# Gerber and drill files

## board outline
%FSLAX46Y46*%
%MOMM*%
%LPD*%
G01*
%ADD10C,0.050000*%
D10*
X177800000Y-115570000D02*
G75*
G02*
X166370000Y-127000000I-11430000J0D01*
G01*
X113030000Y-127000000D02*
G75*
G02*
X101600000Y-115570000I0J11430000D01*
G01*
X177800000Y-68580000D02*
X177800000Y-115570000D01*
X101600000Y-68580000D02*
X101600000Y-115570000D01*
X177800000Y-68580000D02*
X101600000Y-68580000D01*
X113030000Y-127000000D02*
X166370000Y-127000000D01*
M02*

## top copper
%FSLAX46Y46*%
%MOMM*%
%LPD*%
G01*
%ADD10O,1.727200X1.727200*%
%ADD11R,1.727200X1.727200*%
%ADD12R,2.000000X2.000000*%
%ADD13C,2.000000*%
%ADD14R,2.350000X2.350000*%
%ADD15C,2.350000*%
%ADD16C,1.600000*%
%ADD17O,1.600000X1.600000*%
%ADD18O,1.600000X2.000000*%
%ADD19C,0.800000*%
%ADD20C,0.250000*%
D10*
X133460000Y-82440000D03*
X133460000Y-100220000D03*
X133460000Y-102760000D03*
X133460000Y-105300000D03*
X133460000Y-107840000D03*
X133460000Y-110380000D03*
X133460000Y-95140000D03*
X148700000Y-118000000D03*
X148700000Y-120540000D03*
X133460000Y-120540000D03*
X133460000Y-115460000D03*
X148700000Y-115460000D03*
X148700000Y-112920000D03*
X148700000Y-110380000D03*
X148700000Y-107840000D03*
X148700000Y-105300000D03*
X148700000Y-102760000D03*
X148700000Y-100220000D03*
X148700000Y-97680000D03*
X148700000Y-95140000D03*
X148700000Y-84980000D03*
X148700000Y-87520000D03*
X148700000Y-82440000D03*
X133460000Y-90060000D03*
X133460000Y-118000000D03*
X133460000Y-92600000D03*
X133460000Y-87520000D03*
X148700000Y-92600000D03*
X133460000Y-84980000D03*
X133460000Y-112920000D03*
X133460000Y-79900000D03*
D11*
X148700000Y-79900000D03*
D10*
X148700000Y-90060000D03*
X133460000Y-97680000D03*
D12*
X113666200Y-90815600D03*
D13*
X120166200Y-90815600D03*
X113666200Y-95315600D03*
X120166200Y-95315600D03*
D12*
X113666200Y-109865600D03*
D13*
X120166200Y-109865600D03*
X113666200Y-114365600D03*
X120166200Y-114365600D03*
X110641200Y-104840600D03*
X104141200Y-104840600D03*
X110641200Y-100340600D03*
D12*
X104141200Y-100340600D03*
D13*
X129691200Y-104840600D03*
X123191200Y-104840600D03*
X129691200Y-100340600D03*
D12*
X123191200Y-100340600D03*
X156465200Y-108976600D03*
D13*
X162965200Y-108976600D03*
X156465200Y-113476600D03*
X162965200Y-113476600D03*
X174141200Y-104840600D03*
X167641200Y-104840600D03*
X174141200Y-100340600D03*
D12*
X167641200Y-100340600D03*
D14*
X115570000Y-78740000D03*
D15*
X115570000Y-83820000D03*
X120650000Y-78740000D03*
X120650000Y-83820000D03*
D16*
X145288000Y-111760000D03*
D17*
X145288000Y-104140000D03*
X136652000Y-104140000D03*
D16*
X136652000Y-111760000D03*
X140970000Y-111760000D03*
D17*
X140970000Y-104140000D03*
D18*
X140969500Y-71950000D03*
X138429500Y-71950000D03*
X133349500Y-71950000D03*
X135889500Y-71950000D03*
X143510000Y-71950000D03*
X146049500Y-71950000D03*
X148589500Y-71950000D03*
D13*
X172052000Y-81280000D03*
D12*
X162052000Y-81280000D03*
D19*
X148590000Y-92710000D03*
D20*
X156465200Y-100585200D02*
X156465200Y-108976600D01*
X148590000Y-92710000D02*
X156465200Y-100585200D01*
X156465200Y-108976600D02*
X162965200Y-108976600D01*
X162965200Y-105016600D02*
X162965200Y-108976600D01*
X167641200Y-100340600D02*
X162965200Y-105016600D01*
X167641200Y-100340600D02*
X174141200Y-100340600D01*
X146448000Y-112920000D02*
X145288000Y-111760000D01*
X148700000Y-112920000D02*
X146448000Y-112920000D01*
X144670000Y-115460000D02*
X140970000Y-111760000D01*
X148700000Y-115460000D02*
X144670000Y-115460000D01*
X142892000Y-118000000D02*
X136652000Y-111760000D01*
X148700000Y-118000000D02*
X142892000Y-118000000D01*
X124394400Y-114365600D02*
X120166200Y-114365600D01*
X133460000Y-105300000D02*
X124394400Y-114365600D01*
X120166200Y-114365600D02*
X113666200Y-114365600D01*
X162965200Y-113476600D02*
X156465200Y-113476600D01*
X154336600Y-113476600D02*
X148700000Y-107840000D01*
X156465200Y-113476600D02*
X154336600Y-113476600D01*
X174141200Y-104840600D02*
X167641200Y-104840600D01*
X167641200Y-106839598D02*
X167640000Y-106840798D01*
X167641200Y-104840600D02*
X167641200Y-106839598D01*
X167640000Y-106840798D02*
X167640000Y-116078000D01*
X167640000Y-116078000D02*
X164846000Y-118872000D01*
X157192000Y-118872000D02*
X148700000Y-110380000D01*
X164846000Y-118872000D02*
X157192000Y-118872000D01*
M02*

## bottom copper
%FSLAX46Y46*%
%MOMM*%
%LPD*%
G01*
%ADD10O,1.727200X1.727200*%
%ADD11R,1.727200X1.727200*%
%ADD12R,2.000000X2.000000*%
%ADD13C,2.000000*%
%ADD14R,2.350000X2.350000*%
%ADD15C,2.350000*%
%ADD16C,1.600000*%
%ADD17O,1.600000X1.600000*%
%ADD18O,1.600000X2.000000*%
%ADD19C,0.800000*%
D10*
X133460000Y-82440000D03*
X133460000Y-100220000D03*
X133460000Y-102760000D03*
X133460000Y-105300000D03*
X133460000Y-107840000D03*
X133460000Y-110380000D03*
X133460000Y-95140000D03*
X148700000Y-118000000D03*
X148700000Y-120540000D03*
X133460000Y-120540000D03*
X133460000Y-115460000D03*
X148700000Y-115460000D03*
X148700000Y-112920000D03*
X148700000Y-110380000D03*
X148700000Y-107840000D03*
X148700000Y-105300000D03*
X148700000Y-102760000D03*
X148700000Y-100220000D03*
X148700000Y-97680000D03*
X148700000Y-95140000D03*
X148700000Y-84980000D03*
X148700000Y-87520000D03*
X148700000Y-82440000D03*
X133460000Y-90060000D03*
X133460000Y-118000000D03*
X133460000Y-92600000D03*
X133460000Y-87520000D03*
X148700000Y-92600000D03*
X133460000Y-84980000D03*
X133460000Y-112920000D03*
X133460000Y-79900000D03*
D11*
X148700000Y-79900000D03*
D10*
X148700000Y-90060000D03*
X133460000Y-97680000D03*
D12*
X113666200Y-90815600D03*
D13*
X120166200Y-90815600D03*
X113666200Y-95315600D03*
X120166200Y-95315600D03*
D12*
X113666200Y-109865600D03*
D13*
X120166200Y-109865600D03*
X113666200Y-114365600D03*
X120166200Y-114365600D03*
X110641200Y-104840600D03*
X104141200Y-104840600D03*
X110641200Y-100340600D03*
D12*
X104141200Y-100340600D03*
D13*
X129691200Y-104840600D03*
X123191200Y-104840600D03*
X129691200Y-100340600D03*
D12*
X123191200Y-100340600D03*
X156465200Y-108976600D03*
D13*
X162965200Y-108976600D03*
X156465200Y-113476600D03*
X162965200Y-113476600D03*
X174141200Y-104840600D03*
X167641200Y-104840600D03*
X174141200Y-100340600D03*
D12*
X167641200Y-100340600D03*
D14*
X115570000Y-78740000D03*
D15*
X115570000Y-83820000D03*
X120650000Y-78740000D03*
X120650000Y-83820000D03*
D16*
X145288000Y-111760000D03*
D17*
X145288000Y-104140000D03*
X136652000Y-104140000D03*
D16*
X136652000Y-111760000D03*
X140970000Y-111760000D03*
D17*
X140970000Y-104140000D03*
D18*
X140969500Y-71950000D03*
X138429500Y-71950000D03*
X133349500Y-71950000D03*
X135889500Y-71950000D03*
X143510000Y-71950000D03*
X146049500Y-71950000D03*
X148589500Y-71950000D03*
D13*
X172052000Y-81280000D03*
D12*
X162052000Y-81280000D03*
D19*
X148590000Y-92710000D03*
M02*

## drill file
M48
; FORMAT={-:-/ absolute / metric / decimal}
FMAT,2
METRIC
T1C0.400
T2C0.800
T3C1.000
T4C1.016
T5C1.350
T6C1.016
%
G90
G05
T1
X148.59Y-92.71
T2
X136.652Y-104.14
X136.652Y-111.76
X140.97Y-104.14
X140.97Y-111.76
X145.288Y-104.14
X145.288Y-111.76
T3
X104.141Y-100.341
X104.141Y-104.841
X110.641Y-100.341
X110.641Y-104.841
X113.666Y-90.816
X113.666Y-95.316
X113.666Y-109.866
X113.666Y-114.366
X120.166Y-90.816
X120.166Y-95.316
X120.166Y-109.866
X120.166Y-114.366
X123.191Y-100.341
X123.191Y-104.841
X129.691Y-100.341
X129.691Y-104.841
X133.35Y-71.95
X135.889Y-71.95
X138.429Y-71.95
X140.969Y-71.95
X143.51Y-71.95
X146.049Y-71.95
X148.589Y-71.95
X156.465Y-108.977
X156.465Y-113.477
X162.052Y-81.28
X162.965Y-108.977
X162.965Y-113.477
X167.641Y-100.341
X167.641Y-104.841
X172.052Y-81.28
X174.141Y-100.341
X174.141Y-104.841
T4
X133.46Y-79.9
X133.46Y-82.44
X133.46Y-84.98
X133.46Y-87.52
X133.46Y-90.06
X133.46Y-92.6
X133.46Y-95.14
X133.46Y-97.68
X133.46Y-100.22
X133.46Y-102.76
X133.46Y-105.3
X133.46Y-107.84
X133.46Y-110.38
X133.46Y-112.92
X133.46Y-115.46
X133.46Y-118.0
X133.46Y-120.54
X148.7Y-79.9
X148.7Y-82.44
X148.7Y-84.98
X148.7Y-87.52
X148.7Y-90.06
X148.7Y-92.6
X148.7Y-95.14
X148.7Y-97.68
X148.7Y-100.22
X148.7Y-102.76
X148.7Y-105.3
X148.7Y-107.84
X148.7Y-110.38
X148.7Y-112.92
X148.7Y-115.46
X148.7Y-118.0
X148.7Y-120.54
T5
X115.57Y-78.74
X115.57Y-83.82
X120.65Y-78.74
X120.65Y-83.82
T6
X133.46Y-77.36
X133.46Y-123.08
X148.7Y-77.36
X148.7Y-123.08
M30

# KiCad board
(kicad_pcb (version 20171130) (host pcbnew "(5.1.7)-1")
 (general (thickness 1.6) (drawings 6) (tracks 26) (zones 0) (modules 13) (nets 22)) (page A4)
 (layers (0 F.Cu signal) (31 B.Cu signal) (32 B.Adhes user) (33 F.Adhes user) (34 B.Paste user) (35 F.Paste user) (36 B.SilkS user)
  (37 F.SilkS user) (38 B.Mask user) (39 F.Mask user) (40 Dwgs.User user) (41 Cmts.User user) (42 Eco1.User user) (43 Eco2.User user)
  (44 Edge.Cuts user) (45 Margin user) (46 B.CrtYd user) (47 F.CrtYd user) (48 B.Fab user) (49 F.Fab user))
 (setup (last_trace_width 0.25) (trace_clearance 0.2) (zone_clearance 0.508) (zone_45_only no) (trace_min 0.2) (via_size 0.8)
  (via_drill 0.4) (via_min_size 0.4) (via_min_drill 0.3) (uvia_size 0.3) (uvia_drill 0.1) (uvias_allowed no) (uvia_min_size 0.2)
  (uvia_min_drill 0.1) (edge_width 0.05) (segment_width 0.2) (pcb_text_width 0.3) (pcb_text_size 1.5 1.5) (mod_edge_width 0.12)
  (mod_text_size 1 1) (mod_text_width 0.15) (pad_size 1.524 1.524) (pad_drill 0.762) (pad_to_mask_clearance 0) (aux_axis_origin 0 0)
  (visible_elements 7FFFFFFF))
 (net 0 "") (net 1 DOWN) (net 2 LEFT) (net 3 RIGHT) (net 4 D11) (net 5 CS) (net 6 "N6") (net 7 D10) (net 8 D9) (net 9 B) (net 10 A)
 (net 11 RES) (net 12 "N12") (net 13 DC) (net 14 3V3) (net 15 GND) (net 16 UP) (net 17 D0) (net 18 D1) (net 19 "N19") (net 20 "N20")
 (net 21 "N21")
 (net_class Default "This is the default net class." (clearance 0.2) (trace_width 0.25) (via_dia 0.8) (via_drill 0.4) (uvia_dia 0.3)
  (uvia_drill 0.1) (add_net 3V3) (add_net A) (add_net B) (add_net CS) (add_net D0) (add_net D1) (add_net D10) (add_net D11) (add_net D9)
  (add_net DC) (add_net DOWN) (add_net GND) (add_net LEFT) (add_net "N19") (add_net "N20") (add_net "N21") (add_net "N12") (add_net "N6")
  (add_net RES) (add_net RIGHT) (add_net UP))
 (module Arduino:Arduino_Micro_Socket (layer B.Cu) (at 132.08 124.46 90)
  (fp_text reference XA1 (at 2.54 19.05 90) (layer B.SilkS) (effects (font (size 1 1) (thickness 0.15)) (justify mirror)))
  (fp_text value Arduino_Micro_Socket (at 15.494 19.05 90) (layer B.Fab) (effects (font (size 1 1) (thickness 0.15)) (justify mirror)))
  (pad MISO thru_hole oval (at 42.02 1.38 90) (size 1.7272 1.7272) (drill 1.016) (layers *.Cu *.Mask))
  (pad A5 thru_hole oval (at 24.24 1.38 90) (size 1.7272 1.7272) (drill 1.016) (layers *.Cu *.Mask))
  (pad A4 thru_hole oval (at 21.7 1.38 90) (size 1.7272 1.7272) (drill 1.016) (layers *.Cu *.Mask))
  (pad A3 thru_hole oval (at 19.16 1.38 90) (size 1.7272 1.7272) (drill 1.016) (layers *.Cu *.Mask) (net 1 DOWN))
  (pad A2 thru_hole oval (at 16.62 1.38 90) (size 1.7272 1.7272) (drill 1.016) (layers *.Cu *.Mask) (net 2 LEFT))
  (pad A1 thru_hole oval (at 14.08 1.38 90) (size 1.7272 1.7272) (drill 1.016) (layers *.Cu *.Mask) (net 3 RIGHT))
  (pad "" thru_hole oval (at 29.32 1.38 90) (size 1.7272 1.7272) (drill 1.016) (layers *.Cu *.Mask))
  (pad D11 thru_hole oval (at 6.46 16.62 90) (size 1.7272 1.7272) (drill 1.016) (layers *.Cu *.Mask) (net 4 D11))
  (pad D12 thru_hole oval (at 3.92 16.62 90) (size 1.7272 1.7272) (drill 1.016) (layers *.Cu *.Mask) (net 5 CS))
  (pad D13 thru_hole oval (at 3.92 1.38 90) (size 1.7272 1.7272) (drill 1.016) (layers *.Cu *.Mask) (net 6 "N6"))
  (pad AREF thru_hole oval (at 9 1.38 90) (size 1.7272 1.7272) (drill 1.016) (layers *.Cu *.Mask))
  (pad "" np_thru_hole circle (at 1.38 1.38 90) (size 1.016 1.016) (drill 1.016) (layers *.Cu *.Mask))
  (pad D10 thru_hole oval (at 9 16.62 90) (size 1.7272 1.7272) (drill 1.016) (layers *.Cu *.Mask) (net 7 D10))
  (pad D9 thru_hole oval (at 11.54 16.62 90) (size 1.7272 1.7272) (drill 1.016) (layers *.Cu *.Mask) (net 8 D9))
  (pad D8 thru_hole oval (at 14.08 16.62 90) (size 1.7272 1.7272) (drill 1.016) (layers *.Cu *.Mask) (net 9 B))
  (pad D7 thru_hole oval (at 16.62 16.62 90) (size 1.7272 1.7272) (drill 1.016) (layers *.Cu *.Mask) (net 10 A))
  (pad D6 thru_hole oval (at 19.16 16.62 90) (size 1.7272 1.7272) (drill 1.016) (layers *.Cu *.Mask) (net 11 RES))
  (pad D5 thru_hole oval (at 21.7 16.62 90) (size 1.7272 1.7272) (drill 1.016) (layers *.Cu *.Mask) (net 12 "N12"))
  (pad D4 thru_hole oval (at 24.24 16.62 90) (size 1.7272 1.7272) (drill 1.016) (layers *.Cu *.Mask) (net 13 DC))
  (pad D3 thru_hole oval (at 26.78 16.62 90) (size 1.7272 1.7272) (drill 1.016) (layers *.Cu *.Mask))
  (pad D2 thru_hole oval (at 29.32 16.62 90) (size 1.7272 1.7272) (drill 1.016) (layers *.Cu *.Mask))
  (pad D1 thru_hole oval (at 39.48 16.62 90) (size 1.7272 1.7272) (drill 1.016) (layers *.Cu *.Mask))
  (pad D0 thru_hole oval (at 36.94 16.62 90) (size 1.7272 1.7272) (drill 1.016) (layers *.Cu *.Mask))
  (pad SS thru_hole oval (at 42.02 16.62 90) (size 1.7272 1.7272) (drill 1.016) (layers *.Cu *.Mask))
  (pad RST1 thru_hole oval (at 34.4 1.38 90) (size 1.7272 1.7272) (drill 1.016) (layers *.Cu *.Mask))
  (pad 3V3 thru_hole oval (at 6.46 1.38 90) (size 1.7272 1.7272) (drill 1.016) (layers *.Cu *.Mask) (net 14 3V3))
  (pad 5V thru_hole oval (at 31.86 1.38 90) (size 1.7272 1.7272) (drill 1.016) (layers *.Cu *.Mask))
  (pad GND1 thru_hole oval (at 36.94 1.38 90) (size 1.7272 1.7272) (drill 1.016) (layers *.Cu *.Mask) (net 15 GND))
  (pad GND2 thru_hole oval (at 31.86 16.62 90) (size 1.7272 1.7272) (drill 1.016) (layers *.Cu *.Mask) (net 15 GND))
  (pad VIN thru_hole oval (at 39.48 1.38 90) (size 1.7272 1.7272) (drill 1.016) (layers *.Cu *.Mask))
  (pad A0 thru_hole oval (at 11.54 1.38 90) (size 1.7272 1.7272) (drill 1.016) (layers *.Cu *.Mask) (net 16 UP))
  (pad SCK thru_hole oval (at 44.56 1.38 90) (size 1.7272 1.7272) (drill 1.016) (layers *.Cu *.Mask) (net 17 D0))
  (pad MOSI thru_hole rect (at 44.56 16.62 90) (size 1.7272 1.7272) (drill 1.016) (layers *.Cu *.Mask) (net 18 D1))
  (pad RST2 thru_hole oval (at 34.4 16.62 90) (size 1.7272 1.7272) (drill 1.016) (layers *.Cu *.Mask))
  (pad "" thru_hole oval (at 26.78 1.38 90) (size 1.7272 1.7272) (drill 1.016) (layers *.Cu *.Mask))
  (pad "" np_thru_hole circle (at 47.1 1.38 90) (size 1.016 1.016) (drill 1.016) (layers *.Cu *.Mask))
  (pad "" np_thru_hole circle (at 1.38 16.62 90) (size 1.016 1.016) (drill 1.016) (layers *.Cu *.Mask))
  (pad "" np_thru_hole circle (at 47.1 16.62 90) (size 1.016 1.016) (drill 1.016) (layers *.Cu *.Mask)))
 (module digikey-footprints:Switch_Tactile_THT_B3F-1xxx (layer F.Cu) (at 113.665 90.805)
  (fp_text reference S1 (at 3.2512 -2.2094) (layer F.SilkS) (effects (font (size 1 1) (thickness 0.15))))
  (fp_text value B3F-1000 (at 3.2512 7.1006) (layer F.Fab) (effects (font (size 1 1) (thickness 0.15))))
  (pad 1 thru_hole rect (at 0.0012 0.0106) (size 2 2) (drill 1) (layers *.Cu *.Mask) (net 15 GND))
  (pad 2 thru_hole circle (at 6.5012 0.0106) (size 2 2) (drill 1) (layers *.Cu *.Mask) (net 15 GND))
  (pad 3 thru_hole circle (at 0.0012 4.5106) (size 2 2) (drill 1) (layers *.Cu *.Mask) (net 16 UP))
  (pad 4 thru_hole circle (at 6.5012 4.5106) (size 2 2) (drill 1) (layers *.Cu *.Mask) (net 16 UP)))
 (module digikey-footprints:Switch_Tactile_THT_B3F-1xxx (layer F.Cu) (at 113.665 109.855)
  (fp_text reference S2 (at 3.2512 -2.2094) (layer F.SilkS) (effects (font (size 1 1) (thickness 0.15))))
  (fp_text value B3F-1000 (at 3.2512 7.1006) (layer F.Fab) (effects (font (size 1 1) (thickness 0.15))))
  (pad 1 thru_hole rect (at 0.0012 0.0106) (size 2 2) (drill 1) (layers *.Cu *.Mask) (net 15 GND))
  (pad 2 thru_hole circle (at 6.5012 0.0106) (size 2 2) (drill 1) (layers *.Cu *.Mask) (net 15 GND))
  (pad 3 thru_hole circle (at 0.0012 4.5106) (size 2 2) (drill 1) (layers *.Cu *.Mask) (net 1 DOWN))
  (pad 4 thru_hole circle (at 6.5012 4.5106) (size 2 2) (drill 1) (layers *.Cu *.Mask) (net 1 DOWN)))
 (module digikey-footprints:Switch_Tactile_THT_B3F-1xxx (layer F.Cu) (at 104.14 100.33)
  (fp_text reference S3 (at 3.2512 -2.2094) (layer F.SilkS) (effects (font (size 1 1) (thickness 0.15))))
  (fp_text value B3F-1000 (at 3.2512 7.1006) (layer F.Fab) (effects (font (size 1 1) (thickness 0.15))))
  (pad 4 thru_hole circle (at 6.5012 4.5106) (size 2 2) (drill 1) (layers *.Cu *.Mask) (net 2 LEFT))
  (pad 3 thru_hole circle (at 0.0012 4.5106) (size 2 2) (drill 1) (layers *.Cu *.Mask) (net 2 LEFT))
  (pad 2 thru_hole circle (at 6.5012 0.0106) (size 2 2) (drill 1) (layers *.Cu *.Mask) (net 15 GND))
  (pad 1 thru_hole rect (at 0.0012 0.0106) (size 2 2) (drill 1) (layers *.Cu *.Mask) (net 15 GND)))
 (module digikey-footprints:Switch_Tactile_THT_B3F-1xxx (layer F.Cu) (at 123.19 100.33)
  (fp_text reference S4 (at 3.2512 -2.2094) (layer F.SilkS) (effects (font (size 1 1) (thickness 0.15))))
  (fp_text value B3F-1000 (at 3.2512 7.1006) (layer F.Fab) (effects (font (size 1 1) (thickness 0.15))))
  (pad 4 thru_hole circle (at 6.5012 4.5106) (size 2 2) (drill 1) (layers *.Cu *.Mask) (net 3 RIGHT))
  (pad 3 thru_hole circle (at 0.0012 4.5106) (size 2 2) (drill 1) (layers *.Cu *.Mask) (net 3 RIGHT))
  (pad 2 thru_hole circle (at 6.5012 0.0106) (size 2 2) (drill 1) (layers *.Cu *.Mask) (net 15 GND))
  (pad 1 thru_hole rect (at 0.0012 0.0106) (size 2 2) (drill 1) (layers *.Cu *.Mask) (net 15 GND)))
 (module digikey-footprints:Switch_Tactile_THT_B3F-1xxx (layer F.Cu) (at 156.464 108.966)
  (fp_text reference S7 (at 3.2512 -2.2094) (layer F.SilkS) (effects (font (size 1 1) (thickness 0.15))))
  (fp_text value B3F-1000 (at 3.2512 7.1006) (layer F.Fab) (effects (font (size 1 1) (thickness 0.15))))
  (pad 1 thru_hole rect (at 0.0012 0.0106) (size 2 2) (drill 1) (layers *.Cu *.Mask) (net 15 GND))
  (pad 2 thru_hole circle (at 6.5012 0.0106) (size 2 2) (drill 1) (layers *.Cu *.Mask) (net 15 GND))
  (pad 3 thru_hole circle (at 0.0012 4.5106) (size 2 2) (drill 1) (layers *.Cu *.Mask) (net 10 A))
  (pad 4 thru_hole circle (at 6.5012 4.5106) (size 2 2) (drill 1) (layers *.Cu *.Mask) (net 10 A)))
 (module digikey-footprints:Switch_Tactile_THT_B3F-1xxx (layer F.Cu) (at 167.64 100.33)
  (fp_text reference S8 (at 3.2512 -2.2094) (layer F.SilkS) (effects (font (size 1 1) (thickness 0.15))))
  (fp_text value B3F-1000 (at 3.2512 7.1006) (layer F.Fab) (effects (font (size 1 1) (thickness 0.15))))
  (pad 4 thru_hole circle (at 6.5012 4.5106) (size 2 2) (drill 1) (layers *.Cu *.Mask) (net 9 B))
  (pad 3 thru_hole circle (at 0.0012 4.5106) (size 2 2) (drill 1) (layers *.Cu *.Mask) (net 9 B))
  (pad 2 thru_hole circle (at 6.5012 0.0106) (size 2 2) (drill 1) (layers *.Cu *.Mask) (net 15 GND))
  (pad 1 thru_hole rect (at 0.0012 0.0106) (size 2 2) (drill 1) (layers *.Cu *.Mask) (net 15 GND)))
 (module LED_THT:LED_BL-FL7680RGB (layer F.Cu) (at 115.57 78.74)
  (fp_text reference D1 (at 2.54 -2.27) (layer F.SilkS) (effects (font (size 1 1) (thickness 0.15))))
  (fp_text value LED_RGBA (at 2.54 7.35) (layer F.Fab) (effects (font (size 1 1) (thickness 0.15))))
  (pad 1 thru_hole rect (at 0 0) (size 2.35 2.35) (drill 1.35) (layers *.Cu *.Mask) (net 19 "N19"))
  (pad 2 thru_hole circle (at 0 5.08) (size 2.35 2.35) (drill 1.35) (layers *.Cu *.Mask) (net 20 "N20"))
  (pad 4 thru_hole circle (at 5.08 0) (size 2.35 2.35) (drill 1.35) (layers *.Cu *.Mask))
  (pad 3 thru_hole circle (at 5.08 5.08) (size 2.35 2.35) (drill 1.35) (layers *.Cu *.Mask) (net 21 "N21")))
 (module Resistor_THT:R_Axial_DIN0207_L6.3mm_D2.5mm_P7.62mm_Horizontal (layer F.Cu) (at 145.288 111.76 90)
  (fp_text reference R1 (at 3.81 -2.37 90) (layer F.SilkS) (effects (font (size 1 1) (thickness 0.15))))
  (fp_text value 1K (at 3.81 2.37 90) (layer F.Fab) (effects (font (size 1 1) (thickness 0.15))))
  (pad 1 thru_hole circle (at 0 0 90) (size 1.6 1.6) (drill 0.8) (layers *.Cu *.Mask) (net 8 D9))
  (pad 2 thru_hole oval (at 7.62 0 90) (size 1.6 1.6) (drill 0.8) (layers *.Cu *.Mask) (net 21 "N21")))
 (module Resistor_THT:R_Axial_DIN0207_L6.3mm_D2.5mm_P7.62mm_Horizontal (layer F.Cu) (at 136.652 111.76 90)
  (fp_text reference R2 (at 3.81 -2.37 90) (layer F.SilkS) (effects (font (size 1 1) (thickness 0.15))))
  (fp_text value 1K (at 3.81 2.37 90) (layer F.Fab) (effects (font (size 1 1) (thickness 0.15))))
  (pad 2 thru_hole oval (at 7.62 0 90) (size 1.6 1.6) (drill 0.8) (layers *.Cu *.Mask) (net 20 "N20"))
  (pad 1 thru_hole circle (at 0 0 90) (size 1.6 1.6) (drill 0.8) (layers *.Cu *.Mask) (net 4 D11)))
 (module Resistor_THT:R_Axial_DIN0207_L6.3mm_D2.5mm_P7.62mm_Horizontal (layer F.Cu) (at 140.97 111.76 90)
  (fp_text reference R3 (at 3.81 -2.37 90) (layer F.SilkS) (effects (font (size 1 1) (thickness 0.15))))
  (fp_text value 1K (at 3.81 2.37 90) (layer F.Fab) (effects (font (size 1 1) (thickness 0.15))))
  (pad 1 thru_hole circle (at 0 0 90) (size 1.6 1.6) (drill 0.8) (layers *.Cu *.Mask) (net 7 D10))
  (pad 2 thru_hole oval (at 7.62 0 90) (size 1.6 1.6) (drill 0.8) (layers *.Cu *.Mask) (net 19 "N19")))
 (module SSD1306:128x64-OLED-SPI (layer F.Cu) (at 140.97 83.82)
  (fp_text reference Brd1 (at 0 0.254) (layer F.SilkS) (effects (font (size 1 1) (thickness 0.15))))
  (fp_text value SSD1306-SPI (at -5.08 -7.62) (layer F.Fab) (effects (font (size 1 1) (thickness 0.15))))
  (pad 4 thru_hole oval (at -0.0005 -11.87 90) (size 2 1.6) (drill 1) (layers *.Cu *.Mask) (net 18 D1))
  (pad 3 thru_hole oval (at -2.5405 -11.87 90) (size 2 1.6) (drill 1) (layers *.Cu *.Mask) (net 17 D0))
  (pad 1 thru_hole oval (at -7.6205 -11.87 90) (size 2 1.6) (drill 1) (layers *.Cu *.Mask) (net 15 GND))
  (pad 2 thru_hole oval (at -5.0805 -11.87 90) (size 2 1.6) (drill 1) (layers *.Cu *.Mask) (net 14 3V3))
  (pad 5 thru_hole oval (at 2.54 -11.87 90) (size 2 1.6) (drill 1) (layers *.Cu *.Mask) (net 11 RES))
  (pad 6 thru_hole oval (at 5.0795 -11.87 90) (size 2 1.6) (drill 1) (layers *.Cu *.Mask) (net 13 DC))
  (pad 7 thru_hole oval (at 7.6195 -11.87 90) (size 2 1.6) (drill 1) (layers *.Cu *.Mask) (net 5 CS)))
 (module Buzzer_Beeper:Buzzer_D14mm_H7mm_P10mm (layer F.Cu) (at 162.052 81.28)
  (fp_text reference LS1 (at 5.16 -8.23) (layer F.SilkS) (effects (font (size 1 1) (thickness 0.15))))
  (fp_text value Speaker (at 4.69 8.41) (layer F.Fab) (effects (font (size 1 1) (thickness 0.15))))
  (pad 2 thru_hole circle (at 10 0) (size 2 2) (drill 1) (layers *.Cu *.Mask) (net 6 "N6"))
  (pad 1 thru_hole rect (at 0 0) (size 2 2) (drill 1) (layers *.Cu *.Mask) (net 12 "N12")))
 (gr_arc (start 166.37 115.57) (end 166.37 127) (angle -90) (layer Edge.Cuts) (width 0.05))
 (gr_arc (start 113.03 115.57) (end 101.6 115.57) (angle -90) (layer Edge.Cuts) (width 0.05))
 (gr_line (start 177.8 68.58) (end 177.8 115.57) (layer Edge.Cuts) (width 0.05))
 (gr_line (start 101.6 68.58) (end 101.6 115.57) (layer Edge.Cuts) (width 0.05))
 (gr_line (start 177.8 68.58) (end 101.6 68.58) (layer Edge.Cuts) (width 0.05))
 (gr_line (start 113.03 127) (end 166.37 127) (layer Edge.Cuts) (width 0.05))
 (via (at 148.59 92.71) (size 0.8) (drill 0.4) (layers F.Cu B.Cu) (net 15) (status 30))
 (segment (start 156.4652 100.5852) (end 156.4652 108.9766) (width 0.25) (layer F.Cu) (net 15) (status 20))
 (segment (start 148.59 92.71) (end 156.4652 100.5852) (width 0.25) (layer F.Cu) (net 15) (status 10))
 (segment (start 156.4652 108.9766) (end 162.9652 108.9766) (width 0.25) (layer F.Cu) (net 15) (status 30))
 (segment (start 162.9652 105.0166) (end 162.9652 108.9766) (width 0.25) (layer F.Cu) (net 15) (status 20))
 (segment (start 167.6412 100.3406) (end 162.9652 105.0166) (width 0.25) (layer F.Cu) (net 15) (status 10))
 (segment (start 167.6412 100.3406) (end 174.1412 100.3406) (width 0.25) (layer F.Cu) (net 15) (status 30))
 (segment (start 146.448 112.92) (end 145.288 111.76) (width 0.25) (layer F.Cu) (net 8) (status 20))
 (segment (start 148.7 112.92) (end 146.448 112.92) (width 0.25) (layer F.Cu) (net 8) (status 10))
 (segment (start 144.67 115.46) (end 140.97 111.76) (width 0.25) (layer F.Cu) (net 7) (status 20))
 (segment (start 148.7 115.46) (end 144.67 115.46) (width 0.25) (layer F.Cu) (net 7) (status 10))
 (segment (start 142.892 118) (end 136.652 111.76) (width 0.25) (layer F.Cu) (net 4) (status 20))
 (segment (start 148.7 118) (end 142.892 118) (width 0.25) (layer F.Cu) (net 4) (status 10))
 (segment (start 124.3944 114.3656) (end 120.1662 114.3656) (width 0.25) (layer F.Cu) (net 1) (status 20))
 (segment (start 133.46 105.3) (end 124.3944 114.3656) (width 0.25) (layer F.Cu) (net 1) (status 10))
 (segment (start 120.1662 114.3656) (end 113.6662 114.3656) (width 0.25) (layer F.Cu) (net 1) (status 30))
 (segment (start 162.9652 113.4766) (end 156.4652 113.4766) (width 0.25) (layer F.Cu) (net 10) (status 30))
 (segment (start 154.3366 113.4766) (end 148.7 107.84) (width 0.25) (layer F.Cu) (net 10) (status 20))
 (segment (start 156.4652 113.4766) (end 154.3366 113.4766) (width 0.25) (layer F.Cu) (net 10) (status 10))
 (segment (start 174.1412 104.8406) (end 167.6412 104.8406) (width 0.25) (layer F.Cu) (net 9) (status 30))
 (segment (start 167.6412 106.839598) (end 167.64 106.840798) (width 0.25) (layer F.Cu) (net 9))
 (segment (start 167.6412 104.8406) (end 167.6412 106.839598) (width 0.25) (layer F.Cu) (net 9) (status 10))
 (segment (start 167.64 106.840798) (end 167.64 116.078) (width 0.25) (layer F.Cu) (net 9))
 (segment (start 167.64 116.078) (end 164.846 118.872) (width 0.25) (layer F.Cu) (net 9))
 (segment (start 157.192 118.872) (end 148.7 110.38) (width 0.25) (layer F.Cu) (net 9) (status 20))
 (segment (start 164.846 118.872) (end 157.192 118.872) (width 0.25) (layer F.Cu) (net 9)))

